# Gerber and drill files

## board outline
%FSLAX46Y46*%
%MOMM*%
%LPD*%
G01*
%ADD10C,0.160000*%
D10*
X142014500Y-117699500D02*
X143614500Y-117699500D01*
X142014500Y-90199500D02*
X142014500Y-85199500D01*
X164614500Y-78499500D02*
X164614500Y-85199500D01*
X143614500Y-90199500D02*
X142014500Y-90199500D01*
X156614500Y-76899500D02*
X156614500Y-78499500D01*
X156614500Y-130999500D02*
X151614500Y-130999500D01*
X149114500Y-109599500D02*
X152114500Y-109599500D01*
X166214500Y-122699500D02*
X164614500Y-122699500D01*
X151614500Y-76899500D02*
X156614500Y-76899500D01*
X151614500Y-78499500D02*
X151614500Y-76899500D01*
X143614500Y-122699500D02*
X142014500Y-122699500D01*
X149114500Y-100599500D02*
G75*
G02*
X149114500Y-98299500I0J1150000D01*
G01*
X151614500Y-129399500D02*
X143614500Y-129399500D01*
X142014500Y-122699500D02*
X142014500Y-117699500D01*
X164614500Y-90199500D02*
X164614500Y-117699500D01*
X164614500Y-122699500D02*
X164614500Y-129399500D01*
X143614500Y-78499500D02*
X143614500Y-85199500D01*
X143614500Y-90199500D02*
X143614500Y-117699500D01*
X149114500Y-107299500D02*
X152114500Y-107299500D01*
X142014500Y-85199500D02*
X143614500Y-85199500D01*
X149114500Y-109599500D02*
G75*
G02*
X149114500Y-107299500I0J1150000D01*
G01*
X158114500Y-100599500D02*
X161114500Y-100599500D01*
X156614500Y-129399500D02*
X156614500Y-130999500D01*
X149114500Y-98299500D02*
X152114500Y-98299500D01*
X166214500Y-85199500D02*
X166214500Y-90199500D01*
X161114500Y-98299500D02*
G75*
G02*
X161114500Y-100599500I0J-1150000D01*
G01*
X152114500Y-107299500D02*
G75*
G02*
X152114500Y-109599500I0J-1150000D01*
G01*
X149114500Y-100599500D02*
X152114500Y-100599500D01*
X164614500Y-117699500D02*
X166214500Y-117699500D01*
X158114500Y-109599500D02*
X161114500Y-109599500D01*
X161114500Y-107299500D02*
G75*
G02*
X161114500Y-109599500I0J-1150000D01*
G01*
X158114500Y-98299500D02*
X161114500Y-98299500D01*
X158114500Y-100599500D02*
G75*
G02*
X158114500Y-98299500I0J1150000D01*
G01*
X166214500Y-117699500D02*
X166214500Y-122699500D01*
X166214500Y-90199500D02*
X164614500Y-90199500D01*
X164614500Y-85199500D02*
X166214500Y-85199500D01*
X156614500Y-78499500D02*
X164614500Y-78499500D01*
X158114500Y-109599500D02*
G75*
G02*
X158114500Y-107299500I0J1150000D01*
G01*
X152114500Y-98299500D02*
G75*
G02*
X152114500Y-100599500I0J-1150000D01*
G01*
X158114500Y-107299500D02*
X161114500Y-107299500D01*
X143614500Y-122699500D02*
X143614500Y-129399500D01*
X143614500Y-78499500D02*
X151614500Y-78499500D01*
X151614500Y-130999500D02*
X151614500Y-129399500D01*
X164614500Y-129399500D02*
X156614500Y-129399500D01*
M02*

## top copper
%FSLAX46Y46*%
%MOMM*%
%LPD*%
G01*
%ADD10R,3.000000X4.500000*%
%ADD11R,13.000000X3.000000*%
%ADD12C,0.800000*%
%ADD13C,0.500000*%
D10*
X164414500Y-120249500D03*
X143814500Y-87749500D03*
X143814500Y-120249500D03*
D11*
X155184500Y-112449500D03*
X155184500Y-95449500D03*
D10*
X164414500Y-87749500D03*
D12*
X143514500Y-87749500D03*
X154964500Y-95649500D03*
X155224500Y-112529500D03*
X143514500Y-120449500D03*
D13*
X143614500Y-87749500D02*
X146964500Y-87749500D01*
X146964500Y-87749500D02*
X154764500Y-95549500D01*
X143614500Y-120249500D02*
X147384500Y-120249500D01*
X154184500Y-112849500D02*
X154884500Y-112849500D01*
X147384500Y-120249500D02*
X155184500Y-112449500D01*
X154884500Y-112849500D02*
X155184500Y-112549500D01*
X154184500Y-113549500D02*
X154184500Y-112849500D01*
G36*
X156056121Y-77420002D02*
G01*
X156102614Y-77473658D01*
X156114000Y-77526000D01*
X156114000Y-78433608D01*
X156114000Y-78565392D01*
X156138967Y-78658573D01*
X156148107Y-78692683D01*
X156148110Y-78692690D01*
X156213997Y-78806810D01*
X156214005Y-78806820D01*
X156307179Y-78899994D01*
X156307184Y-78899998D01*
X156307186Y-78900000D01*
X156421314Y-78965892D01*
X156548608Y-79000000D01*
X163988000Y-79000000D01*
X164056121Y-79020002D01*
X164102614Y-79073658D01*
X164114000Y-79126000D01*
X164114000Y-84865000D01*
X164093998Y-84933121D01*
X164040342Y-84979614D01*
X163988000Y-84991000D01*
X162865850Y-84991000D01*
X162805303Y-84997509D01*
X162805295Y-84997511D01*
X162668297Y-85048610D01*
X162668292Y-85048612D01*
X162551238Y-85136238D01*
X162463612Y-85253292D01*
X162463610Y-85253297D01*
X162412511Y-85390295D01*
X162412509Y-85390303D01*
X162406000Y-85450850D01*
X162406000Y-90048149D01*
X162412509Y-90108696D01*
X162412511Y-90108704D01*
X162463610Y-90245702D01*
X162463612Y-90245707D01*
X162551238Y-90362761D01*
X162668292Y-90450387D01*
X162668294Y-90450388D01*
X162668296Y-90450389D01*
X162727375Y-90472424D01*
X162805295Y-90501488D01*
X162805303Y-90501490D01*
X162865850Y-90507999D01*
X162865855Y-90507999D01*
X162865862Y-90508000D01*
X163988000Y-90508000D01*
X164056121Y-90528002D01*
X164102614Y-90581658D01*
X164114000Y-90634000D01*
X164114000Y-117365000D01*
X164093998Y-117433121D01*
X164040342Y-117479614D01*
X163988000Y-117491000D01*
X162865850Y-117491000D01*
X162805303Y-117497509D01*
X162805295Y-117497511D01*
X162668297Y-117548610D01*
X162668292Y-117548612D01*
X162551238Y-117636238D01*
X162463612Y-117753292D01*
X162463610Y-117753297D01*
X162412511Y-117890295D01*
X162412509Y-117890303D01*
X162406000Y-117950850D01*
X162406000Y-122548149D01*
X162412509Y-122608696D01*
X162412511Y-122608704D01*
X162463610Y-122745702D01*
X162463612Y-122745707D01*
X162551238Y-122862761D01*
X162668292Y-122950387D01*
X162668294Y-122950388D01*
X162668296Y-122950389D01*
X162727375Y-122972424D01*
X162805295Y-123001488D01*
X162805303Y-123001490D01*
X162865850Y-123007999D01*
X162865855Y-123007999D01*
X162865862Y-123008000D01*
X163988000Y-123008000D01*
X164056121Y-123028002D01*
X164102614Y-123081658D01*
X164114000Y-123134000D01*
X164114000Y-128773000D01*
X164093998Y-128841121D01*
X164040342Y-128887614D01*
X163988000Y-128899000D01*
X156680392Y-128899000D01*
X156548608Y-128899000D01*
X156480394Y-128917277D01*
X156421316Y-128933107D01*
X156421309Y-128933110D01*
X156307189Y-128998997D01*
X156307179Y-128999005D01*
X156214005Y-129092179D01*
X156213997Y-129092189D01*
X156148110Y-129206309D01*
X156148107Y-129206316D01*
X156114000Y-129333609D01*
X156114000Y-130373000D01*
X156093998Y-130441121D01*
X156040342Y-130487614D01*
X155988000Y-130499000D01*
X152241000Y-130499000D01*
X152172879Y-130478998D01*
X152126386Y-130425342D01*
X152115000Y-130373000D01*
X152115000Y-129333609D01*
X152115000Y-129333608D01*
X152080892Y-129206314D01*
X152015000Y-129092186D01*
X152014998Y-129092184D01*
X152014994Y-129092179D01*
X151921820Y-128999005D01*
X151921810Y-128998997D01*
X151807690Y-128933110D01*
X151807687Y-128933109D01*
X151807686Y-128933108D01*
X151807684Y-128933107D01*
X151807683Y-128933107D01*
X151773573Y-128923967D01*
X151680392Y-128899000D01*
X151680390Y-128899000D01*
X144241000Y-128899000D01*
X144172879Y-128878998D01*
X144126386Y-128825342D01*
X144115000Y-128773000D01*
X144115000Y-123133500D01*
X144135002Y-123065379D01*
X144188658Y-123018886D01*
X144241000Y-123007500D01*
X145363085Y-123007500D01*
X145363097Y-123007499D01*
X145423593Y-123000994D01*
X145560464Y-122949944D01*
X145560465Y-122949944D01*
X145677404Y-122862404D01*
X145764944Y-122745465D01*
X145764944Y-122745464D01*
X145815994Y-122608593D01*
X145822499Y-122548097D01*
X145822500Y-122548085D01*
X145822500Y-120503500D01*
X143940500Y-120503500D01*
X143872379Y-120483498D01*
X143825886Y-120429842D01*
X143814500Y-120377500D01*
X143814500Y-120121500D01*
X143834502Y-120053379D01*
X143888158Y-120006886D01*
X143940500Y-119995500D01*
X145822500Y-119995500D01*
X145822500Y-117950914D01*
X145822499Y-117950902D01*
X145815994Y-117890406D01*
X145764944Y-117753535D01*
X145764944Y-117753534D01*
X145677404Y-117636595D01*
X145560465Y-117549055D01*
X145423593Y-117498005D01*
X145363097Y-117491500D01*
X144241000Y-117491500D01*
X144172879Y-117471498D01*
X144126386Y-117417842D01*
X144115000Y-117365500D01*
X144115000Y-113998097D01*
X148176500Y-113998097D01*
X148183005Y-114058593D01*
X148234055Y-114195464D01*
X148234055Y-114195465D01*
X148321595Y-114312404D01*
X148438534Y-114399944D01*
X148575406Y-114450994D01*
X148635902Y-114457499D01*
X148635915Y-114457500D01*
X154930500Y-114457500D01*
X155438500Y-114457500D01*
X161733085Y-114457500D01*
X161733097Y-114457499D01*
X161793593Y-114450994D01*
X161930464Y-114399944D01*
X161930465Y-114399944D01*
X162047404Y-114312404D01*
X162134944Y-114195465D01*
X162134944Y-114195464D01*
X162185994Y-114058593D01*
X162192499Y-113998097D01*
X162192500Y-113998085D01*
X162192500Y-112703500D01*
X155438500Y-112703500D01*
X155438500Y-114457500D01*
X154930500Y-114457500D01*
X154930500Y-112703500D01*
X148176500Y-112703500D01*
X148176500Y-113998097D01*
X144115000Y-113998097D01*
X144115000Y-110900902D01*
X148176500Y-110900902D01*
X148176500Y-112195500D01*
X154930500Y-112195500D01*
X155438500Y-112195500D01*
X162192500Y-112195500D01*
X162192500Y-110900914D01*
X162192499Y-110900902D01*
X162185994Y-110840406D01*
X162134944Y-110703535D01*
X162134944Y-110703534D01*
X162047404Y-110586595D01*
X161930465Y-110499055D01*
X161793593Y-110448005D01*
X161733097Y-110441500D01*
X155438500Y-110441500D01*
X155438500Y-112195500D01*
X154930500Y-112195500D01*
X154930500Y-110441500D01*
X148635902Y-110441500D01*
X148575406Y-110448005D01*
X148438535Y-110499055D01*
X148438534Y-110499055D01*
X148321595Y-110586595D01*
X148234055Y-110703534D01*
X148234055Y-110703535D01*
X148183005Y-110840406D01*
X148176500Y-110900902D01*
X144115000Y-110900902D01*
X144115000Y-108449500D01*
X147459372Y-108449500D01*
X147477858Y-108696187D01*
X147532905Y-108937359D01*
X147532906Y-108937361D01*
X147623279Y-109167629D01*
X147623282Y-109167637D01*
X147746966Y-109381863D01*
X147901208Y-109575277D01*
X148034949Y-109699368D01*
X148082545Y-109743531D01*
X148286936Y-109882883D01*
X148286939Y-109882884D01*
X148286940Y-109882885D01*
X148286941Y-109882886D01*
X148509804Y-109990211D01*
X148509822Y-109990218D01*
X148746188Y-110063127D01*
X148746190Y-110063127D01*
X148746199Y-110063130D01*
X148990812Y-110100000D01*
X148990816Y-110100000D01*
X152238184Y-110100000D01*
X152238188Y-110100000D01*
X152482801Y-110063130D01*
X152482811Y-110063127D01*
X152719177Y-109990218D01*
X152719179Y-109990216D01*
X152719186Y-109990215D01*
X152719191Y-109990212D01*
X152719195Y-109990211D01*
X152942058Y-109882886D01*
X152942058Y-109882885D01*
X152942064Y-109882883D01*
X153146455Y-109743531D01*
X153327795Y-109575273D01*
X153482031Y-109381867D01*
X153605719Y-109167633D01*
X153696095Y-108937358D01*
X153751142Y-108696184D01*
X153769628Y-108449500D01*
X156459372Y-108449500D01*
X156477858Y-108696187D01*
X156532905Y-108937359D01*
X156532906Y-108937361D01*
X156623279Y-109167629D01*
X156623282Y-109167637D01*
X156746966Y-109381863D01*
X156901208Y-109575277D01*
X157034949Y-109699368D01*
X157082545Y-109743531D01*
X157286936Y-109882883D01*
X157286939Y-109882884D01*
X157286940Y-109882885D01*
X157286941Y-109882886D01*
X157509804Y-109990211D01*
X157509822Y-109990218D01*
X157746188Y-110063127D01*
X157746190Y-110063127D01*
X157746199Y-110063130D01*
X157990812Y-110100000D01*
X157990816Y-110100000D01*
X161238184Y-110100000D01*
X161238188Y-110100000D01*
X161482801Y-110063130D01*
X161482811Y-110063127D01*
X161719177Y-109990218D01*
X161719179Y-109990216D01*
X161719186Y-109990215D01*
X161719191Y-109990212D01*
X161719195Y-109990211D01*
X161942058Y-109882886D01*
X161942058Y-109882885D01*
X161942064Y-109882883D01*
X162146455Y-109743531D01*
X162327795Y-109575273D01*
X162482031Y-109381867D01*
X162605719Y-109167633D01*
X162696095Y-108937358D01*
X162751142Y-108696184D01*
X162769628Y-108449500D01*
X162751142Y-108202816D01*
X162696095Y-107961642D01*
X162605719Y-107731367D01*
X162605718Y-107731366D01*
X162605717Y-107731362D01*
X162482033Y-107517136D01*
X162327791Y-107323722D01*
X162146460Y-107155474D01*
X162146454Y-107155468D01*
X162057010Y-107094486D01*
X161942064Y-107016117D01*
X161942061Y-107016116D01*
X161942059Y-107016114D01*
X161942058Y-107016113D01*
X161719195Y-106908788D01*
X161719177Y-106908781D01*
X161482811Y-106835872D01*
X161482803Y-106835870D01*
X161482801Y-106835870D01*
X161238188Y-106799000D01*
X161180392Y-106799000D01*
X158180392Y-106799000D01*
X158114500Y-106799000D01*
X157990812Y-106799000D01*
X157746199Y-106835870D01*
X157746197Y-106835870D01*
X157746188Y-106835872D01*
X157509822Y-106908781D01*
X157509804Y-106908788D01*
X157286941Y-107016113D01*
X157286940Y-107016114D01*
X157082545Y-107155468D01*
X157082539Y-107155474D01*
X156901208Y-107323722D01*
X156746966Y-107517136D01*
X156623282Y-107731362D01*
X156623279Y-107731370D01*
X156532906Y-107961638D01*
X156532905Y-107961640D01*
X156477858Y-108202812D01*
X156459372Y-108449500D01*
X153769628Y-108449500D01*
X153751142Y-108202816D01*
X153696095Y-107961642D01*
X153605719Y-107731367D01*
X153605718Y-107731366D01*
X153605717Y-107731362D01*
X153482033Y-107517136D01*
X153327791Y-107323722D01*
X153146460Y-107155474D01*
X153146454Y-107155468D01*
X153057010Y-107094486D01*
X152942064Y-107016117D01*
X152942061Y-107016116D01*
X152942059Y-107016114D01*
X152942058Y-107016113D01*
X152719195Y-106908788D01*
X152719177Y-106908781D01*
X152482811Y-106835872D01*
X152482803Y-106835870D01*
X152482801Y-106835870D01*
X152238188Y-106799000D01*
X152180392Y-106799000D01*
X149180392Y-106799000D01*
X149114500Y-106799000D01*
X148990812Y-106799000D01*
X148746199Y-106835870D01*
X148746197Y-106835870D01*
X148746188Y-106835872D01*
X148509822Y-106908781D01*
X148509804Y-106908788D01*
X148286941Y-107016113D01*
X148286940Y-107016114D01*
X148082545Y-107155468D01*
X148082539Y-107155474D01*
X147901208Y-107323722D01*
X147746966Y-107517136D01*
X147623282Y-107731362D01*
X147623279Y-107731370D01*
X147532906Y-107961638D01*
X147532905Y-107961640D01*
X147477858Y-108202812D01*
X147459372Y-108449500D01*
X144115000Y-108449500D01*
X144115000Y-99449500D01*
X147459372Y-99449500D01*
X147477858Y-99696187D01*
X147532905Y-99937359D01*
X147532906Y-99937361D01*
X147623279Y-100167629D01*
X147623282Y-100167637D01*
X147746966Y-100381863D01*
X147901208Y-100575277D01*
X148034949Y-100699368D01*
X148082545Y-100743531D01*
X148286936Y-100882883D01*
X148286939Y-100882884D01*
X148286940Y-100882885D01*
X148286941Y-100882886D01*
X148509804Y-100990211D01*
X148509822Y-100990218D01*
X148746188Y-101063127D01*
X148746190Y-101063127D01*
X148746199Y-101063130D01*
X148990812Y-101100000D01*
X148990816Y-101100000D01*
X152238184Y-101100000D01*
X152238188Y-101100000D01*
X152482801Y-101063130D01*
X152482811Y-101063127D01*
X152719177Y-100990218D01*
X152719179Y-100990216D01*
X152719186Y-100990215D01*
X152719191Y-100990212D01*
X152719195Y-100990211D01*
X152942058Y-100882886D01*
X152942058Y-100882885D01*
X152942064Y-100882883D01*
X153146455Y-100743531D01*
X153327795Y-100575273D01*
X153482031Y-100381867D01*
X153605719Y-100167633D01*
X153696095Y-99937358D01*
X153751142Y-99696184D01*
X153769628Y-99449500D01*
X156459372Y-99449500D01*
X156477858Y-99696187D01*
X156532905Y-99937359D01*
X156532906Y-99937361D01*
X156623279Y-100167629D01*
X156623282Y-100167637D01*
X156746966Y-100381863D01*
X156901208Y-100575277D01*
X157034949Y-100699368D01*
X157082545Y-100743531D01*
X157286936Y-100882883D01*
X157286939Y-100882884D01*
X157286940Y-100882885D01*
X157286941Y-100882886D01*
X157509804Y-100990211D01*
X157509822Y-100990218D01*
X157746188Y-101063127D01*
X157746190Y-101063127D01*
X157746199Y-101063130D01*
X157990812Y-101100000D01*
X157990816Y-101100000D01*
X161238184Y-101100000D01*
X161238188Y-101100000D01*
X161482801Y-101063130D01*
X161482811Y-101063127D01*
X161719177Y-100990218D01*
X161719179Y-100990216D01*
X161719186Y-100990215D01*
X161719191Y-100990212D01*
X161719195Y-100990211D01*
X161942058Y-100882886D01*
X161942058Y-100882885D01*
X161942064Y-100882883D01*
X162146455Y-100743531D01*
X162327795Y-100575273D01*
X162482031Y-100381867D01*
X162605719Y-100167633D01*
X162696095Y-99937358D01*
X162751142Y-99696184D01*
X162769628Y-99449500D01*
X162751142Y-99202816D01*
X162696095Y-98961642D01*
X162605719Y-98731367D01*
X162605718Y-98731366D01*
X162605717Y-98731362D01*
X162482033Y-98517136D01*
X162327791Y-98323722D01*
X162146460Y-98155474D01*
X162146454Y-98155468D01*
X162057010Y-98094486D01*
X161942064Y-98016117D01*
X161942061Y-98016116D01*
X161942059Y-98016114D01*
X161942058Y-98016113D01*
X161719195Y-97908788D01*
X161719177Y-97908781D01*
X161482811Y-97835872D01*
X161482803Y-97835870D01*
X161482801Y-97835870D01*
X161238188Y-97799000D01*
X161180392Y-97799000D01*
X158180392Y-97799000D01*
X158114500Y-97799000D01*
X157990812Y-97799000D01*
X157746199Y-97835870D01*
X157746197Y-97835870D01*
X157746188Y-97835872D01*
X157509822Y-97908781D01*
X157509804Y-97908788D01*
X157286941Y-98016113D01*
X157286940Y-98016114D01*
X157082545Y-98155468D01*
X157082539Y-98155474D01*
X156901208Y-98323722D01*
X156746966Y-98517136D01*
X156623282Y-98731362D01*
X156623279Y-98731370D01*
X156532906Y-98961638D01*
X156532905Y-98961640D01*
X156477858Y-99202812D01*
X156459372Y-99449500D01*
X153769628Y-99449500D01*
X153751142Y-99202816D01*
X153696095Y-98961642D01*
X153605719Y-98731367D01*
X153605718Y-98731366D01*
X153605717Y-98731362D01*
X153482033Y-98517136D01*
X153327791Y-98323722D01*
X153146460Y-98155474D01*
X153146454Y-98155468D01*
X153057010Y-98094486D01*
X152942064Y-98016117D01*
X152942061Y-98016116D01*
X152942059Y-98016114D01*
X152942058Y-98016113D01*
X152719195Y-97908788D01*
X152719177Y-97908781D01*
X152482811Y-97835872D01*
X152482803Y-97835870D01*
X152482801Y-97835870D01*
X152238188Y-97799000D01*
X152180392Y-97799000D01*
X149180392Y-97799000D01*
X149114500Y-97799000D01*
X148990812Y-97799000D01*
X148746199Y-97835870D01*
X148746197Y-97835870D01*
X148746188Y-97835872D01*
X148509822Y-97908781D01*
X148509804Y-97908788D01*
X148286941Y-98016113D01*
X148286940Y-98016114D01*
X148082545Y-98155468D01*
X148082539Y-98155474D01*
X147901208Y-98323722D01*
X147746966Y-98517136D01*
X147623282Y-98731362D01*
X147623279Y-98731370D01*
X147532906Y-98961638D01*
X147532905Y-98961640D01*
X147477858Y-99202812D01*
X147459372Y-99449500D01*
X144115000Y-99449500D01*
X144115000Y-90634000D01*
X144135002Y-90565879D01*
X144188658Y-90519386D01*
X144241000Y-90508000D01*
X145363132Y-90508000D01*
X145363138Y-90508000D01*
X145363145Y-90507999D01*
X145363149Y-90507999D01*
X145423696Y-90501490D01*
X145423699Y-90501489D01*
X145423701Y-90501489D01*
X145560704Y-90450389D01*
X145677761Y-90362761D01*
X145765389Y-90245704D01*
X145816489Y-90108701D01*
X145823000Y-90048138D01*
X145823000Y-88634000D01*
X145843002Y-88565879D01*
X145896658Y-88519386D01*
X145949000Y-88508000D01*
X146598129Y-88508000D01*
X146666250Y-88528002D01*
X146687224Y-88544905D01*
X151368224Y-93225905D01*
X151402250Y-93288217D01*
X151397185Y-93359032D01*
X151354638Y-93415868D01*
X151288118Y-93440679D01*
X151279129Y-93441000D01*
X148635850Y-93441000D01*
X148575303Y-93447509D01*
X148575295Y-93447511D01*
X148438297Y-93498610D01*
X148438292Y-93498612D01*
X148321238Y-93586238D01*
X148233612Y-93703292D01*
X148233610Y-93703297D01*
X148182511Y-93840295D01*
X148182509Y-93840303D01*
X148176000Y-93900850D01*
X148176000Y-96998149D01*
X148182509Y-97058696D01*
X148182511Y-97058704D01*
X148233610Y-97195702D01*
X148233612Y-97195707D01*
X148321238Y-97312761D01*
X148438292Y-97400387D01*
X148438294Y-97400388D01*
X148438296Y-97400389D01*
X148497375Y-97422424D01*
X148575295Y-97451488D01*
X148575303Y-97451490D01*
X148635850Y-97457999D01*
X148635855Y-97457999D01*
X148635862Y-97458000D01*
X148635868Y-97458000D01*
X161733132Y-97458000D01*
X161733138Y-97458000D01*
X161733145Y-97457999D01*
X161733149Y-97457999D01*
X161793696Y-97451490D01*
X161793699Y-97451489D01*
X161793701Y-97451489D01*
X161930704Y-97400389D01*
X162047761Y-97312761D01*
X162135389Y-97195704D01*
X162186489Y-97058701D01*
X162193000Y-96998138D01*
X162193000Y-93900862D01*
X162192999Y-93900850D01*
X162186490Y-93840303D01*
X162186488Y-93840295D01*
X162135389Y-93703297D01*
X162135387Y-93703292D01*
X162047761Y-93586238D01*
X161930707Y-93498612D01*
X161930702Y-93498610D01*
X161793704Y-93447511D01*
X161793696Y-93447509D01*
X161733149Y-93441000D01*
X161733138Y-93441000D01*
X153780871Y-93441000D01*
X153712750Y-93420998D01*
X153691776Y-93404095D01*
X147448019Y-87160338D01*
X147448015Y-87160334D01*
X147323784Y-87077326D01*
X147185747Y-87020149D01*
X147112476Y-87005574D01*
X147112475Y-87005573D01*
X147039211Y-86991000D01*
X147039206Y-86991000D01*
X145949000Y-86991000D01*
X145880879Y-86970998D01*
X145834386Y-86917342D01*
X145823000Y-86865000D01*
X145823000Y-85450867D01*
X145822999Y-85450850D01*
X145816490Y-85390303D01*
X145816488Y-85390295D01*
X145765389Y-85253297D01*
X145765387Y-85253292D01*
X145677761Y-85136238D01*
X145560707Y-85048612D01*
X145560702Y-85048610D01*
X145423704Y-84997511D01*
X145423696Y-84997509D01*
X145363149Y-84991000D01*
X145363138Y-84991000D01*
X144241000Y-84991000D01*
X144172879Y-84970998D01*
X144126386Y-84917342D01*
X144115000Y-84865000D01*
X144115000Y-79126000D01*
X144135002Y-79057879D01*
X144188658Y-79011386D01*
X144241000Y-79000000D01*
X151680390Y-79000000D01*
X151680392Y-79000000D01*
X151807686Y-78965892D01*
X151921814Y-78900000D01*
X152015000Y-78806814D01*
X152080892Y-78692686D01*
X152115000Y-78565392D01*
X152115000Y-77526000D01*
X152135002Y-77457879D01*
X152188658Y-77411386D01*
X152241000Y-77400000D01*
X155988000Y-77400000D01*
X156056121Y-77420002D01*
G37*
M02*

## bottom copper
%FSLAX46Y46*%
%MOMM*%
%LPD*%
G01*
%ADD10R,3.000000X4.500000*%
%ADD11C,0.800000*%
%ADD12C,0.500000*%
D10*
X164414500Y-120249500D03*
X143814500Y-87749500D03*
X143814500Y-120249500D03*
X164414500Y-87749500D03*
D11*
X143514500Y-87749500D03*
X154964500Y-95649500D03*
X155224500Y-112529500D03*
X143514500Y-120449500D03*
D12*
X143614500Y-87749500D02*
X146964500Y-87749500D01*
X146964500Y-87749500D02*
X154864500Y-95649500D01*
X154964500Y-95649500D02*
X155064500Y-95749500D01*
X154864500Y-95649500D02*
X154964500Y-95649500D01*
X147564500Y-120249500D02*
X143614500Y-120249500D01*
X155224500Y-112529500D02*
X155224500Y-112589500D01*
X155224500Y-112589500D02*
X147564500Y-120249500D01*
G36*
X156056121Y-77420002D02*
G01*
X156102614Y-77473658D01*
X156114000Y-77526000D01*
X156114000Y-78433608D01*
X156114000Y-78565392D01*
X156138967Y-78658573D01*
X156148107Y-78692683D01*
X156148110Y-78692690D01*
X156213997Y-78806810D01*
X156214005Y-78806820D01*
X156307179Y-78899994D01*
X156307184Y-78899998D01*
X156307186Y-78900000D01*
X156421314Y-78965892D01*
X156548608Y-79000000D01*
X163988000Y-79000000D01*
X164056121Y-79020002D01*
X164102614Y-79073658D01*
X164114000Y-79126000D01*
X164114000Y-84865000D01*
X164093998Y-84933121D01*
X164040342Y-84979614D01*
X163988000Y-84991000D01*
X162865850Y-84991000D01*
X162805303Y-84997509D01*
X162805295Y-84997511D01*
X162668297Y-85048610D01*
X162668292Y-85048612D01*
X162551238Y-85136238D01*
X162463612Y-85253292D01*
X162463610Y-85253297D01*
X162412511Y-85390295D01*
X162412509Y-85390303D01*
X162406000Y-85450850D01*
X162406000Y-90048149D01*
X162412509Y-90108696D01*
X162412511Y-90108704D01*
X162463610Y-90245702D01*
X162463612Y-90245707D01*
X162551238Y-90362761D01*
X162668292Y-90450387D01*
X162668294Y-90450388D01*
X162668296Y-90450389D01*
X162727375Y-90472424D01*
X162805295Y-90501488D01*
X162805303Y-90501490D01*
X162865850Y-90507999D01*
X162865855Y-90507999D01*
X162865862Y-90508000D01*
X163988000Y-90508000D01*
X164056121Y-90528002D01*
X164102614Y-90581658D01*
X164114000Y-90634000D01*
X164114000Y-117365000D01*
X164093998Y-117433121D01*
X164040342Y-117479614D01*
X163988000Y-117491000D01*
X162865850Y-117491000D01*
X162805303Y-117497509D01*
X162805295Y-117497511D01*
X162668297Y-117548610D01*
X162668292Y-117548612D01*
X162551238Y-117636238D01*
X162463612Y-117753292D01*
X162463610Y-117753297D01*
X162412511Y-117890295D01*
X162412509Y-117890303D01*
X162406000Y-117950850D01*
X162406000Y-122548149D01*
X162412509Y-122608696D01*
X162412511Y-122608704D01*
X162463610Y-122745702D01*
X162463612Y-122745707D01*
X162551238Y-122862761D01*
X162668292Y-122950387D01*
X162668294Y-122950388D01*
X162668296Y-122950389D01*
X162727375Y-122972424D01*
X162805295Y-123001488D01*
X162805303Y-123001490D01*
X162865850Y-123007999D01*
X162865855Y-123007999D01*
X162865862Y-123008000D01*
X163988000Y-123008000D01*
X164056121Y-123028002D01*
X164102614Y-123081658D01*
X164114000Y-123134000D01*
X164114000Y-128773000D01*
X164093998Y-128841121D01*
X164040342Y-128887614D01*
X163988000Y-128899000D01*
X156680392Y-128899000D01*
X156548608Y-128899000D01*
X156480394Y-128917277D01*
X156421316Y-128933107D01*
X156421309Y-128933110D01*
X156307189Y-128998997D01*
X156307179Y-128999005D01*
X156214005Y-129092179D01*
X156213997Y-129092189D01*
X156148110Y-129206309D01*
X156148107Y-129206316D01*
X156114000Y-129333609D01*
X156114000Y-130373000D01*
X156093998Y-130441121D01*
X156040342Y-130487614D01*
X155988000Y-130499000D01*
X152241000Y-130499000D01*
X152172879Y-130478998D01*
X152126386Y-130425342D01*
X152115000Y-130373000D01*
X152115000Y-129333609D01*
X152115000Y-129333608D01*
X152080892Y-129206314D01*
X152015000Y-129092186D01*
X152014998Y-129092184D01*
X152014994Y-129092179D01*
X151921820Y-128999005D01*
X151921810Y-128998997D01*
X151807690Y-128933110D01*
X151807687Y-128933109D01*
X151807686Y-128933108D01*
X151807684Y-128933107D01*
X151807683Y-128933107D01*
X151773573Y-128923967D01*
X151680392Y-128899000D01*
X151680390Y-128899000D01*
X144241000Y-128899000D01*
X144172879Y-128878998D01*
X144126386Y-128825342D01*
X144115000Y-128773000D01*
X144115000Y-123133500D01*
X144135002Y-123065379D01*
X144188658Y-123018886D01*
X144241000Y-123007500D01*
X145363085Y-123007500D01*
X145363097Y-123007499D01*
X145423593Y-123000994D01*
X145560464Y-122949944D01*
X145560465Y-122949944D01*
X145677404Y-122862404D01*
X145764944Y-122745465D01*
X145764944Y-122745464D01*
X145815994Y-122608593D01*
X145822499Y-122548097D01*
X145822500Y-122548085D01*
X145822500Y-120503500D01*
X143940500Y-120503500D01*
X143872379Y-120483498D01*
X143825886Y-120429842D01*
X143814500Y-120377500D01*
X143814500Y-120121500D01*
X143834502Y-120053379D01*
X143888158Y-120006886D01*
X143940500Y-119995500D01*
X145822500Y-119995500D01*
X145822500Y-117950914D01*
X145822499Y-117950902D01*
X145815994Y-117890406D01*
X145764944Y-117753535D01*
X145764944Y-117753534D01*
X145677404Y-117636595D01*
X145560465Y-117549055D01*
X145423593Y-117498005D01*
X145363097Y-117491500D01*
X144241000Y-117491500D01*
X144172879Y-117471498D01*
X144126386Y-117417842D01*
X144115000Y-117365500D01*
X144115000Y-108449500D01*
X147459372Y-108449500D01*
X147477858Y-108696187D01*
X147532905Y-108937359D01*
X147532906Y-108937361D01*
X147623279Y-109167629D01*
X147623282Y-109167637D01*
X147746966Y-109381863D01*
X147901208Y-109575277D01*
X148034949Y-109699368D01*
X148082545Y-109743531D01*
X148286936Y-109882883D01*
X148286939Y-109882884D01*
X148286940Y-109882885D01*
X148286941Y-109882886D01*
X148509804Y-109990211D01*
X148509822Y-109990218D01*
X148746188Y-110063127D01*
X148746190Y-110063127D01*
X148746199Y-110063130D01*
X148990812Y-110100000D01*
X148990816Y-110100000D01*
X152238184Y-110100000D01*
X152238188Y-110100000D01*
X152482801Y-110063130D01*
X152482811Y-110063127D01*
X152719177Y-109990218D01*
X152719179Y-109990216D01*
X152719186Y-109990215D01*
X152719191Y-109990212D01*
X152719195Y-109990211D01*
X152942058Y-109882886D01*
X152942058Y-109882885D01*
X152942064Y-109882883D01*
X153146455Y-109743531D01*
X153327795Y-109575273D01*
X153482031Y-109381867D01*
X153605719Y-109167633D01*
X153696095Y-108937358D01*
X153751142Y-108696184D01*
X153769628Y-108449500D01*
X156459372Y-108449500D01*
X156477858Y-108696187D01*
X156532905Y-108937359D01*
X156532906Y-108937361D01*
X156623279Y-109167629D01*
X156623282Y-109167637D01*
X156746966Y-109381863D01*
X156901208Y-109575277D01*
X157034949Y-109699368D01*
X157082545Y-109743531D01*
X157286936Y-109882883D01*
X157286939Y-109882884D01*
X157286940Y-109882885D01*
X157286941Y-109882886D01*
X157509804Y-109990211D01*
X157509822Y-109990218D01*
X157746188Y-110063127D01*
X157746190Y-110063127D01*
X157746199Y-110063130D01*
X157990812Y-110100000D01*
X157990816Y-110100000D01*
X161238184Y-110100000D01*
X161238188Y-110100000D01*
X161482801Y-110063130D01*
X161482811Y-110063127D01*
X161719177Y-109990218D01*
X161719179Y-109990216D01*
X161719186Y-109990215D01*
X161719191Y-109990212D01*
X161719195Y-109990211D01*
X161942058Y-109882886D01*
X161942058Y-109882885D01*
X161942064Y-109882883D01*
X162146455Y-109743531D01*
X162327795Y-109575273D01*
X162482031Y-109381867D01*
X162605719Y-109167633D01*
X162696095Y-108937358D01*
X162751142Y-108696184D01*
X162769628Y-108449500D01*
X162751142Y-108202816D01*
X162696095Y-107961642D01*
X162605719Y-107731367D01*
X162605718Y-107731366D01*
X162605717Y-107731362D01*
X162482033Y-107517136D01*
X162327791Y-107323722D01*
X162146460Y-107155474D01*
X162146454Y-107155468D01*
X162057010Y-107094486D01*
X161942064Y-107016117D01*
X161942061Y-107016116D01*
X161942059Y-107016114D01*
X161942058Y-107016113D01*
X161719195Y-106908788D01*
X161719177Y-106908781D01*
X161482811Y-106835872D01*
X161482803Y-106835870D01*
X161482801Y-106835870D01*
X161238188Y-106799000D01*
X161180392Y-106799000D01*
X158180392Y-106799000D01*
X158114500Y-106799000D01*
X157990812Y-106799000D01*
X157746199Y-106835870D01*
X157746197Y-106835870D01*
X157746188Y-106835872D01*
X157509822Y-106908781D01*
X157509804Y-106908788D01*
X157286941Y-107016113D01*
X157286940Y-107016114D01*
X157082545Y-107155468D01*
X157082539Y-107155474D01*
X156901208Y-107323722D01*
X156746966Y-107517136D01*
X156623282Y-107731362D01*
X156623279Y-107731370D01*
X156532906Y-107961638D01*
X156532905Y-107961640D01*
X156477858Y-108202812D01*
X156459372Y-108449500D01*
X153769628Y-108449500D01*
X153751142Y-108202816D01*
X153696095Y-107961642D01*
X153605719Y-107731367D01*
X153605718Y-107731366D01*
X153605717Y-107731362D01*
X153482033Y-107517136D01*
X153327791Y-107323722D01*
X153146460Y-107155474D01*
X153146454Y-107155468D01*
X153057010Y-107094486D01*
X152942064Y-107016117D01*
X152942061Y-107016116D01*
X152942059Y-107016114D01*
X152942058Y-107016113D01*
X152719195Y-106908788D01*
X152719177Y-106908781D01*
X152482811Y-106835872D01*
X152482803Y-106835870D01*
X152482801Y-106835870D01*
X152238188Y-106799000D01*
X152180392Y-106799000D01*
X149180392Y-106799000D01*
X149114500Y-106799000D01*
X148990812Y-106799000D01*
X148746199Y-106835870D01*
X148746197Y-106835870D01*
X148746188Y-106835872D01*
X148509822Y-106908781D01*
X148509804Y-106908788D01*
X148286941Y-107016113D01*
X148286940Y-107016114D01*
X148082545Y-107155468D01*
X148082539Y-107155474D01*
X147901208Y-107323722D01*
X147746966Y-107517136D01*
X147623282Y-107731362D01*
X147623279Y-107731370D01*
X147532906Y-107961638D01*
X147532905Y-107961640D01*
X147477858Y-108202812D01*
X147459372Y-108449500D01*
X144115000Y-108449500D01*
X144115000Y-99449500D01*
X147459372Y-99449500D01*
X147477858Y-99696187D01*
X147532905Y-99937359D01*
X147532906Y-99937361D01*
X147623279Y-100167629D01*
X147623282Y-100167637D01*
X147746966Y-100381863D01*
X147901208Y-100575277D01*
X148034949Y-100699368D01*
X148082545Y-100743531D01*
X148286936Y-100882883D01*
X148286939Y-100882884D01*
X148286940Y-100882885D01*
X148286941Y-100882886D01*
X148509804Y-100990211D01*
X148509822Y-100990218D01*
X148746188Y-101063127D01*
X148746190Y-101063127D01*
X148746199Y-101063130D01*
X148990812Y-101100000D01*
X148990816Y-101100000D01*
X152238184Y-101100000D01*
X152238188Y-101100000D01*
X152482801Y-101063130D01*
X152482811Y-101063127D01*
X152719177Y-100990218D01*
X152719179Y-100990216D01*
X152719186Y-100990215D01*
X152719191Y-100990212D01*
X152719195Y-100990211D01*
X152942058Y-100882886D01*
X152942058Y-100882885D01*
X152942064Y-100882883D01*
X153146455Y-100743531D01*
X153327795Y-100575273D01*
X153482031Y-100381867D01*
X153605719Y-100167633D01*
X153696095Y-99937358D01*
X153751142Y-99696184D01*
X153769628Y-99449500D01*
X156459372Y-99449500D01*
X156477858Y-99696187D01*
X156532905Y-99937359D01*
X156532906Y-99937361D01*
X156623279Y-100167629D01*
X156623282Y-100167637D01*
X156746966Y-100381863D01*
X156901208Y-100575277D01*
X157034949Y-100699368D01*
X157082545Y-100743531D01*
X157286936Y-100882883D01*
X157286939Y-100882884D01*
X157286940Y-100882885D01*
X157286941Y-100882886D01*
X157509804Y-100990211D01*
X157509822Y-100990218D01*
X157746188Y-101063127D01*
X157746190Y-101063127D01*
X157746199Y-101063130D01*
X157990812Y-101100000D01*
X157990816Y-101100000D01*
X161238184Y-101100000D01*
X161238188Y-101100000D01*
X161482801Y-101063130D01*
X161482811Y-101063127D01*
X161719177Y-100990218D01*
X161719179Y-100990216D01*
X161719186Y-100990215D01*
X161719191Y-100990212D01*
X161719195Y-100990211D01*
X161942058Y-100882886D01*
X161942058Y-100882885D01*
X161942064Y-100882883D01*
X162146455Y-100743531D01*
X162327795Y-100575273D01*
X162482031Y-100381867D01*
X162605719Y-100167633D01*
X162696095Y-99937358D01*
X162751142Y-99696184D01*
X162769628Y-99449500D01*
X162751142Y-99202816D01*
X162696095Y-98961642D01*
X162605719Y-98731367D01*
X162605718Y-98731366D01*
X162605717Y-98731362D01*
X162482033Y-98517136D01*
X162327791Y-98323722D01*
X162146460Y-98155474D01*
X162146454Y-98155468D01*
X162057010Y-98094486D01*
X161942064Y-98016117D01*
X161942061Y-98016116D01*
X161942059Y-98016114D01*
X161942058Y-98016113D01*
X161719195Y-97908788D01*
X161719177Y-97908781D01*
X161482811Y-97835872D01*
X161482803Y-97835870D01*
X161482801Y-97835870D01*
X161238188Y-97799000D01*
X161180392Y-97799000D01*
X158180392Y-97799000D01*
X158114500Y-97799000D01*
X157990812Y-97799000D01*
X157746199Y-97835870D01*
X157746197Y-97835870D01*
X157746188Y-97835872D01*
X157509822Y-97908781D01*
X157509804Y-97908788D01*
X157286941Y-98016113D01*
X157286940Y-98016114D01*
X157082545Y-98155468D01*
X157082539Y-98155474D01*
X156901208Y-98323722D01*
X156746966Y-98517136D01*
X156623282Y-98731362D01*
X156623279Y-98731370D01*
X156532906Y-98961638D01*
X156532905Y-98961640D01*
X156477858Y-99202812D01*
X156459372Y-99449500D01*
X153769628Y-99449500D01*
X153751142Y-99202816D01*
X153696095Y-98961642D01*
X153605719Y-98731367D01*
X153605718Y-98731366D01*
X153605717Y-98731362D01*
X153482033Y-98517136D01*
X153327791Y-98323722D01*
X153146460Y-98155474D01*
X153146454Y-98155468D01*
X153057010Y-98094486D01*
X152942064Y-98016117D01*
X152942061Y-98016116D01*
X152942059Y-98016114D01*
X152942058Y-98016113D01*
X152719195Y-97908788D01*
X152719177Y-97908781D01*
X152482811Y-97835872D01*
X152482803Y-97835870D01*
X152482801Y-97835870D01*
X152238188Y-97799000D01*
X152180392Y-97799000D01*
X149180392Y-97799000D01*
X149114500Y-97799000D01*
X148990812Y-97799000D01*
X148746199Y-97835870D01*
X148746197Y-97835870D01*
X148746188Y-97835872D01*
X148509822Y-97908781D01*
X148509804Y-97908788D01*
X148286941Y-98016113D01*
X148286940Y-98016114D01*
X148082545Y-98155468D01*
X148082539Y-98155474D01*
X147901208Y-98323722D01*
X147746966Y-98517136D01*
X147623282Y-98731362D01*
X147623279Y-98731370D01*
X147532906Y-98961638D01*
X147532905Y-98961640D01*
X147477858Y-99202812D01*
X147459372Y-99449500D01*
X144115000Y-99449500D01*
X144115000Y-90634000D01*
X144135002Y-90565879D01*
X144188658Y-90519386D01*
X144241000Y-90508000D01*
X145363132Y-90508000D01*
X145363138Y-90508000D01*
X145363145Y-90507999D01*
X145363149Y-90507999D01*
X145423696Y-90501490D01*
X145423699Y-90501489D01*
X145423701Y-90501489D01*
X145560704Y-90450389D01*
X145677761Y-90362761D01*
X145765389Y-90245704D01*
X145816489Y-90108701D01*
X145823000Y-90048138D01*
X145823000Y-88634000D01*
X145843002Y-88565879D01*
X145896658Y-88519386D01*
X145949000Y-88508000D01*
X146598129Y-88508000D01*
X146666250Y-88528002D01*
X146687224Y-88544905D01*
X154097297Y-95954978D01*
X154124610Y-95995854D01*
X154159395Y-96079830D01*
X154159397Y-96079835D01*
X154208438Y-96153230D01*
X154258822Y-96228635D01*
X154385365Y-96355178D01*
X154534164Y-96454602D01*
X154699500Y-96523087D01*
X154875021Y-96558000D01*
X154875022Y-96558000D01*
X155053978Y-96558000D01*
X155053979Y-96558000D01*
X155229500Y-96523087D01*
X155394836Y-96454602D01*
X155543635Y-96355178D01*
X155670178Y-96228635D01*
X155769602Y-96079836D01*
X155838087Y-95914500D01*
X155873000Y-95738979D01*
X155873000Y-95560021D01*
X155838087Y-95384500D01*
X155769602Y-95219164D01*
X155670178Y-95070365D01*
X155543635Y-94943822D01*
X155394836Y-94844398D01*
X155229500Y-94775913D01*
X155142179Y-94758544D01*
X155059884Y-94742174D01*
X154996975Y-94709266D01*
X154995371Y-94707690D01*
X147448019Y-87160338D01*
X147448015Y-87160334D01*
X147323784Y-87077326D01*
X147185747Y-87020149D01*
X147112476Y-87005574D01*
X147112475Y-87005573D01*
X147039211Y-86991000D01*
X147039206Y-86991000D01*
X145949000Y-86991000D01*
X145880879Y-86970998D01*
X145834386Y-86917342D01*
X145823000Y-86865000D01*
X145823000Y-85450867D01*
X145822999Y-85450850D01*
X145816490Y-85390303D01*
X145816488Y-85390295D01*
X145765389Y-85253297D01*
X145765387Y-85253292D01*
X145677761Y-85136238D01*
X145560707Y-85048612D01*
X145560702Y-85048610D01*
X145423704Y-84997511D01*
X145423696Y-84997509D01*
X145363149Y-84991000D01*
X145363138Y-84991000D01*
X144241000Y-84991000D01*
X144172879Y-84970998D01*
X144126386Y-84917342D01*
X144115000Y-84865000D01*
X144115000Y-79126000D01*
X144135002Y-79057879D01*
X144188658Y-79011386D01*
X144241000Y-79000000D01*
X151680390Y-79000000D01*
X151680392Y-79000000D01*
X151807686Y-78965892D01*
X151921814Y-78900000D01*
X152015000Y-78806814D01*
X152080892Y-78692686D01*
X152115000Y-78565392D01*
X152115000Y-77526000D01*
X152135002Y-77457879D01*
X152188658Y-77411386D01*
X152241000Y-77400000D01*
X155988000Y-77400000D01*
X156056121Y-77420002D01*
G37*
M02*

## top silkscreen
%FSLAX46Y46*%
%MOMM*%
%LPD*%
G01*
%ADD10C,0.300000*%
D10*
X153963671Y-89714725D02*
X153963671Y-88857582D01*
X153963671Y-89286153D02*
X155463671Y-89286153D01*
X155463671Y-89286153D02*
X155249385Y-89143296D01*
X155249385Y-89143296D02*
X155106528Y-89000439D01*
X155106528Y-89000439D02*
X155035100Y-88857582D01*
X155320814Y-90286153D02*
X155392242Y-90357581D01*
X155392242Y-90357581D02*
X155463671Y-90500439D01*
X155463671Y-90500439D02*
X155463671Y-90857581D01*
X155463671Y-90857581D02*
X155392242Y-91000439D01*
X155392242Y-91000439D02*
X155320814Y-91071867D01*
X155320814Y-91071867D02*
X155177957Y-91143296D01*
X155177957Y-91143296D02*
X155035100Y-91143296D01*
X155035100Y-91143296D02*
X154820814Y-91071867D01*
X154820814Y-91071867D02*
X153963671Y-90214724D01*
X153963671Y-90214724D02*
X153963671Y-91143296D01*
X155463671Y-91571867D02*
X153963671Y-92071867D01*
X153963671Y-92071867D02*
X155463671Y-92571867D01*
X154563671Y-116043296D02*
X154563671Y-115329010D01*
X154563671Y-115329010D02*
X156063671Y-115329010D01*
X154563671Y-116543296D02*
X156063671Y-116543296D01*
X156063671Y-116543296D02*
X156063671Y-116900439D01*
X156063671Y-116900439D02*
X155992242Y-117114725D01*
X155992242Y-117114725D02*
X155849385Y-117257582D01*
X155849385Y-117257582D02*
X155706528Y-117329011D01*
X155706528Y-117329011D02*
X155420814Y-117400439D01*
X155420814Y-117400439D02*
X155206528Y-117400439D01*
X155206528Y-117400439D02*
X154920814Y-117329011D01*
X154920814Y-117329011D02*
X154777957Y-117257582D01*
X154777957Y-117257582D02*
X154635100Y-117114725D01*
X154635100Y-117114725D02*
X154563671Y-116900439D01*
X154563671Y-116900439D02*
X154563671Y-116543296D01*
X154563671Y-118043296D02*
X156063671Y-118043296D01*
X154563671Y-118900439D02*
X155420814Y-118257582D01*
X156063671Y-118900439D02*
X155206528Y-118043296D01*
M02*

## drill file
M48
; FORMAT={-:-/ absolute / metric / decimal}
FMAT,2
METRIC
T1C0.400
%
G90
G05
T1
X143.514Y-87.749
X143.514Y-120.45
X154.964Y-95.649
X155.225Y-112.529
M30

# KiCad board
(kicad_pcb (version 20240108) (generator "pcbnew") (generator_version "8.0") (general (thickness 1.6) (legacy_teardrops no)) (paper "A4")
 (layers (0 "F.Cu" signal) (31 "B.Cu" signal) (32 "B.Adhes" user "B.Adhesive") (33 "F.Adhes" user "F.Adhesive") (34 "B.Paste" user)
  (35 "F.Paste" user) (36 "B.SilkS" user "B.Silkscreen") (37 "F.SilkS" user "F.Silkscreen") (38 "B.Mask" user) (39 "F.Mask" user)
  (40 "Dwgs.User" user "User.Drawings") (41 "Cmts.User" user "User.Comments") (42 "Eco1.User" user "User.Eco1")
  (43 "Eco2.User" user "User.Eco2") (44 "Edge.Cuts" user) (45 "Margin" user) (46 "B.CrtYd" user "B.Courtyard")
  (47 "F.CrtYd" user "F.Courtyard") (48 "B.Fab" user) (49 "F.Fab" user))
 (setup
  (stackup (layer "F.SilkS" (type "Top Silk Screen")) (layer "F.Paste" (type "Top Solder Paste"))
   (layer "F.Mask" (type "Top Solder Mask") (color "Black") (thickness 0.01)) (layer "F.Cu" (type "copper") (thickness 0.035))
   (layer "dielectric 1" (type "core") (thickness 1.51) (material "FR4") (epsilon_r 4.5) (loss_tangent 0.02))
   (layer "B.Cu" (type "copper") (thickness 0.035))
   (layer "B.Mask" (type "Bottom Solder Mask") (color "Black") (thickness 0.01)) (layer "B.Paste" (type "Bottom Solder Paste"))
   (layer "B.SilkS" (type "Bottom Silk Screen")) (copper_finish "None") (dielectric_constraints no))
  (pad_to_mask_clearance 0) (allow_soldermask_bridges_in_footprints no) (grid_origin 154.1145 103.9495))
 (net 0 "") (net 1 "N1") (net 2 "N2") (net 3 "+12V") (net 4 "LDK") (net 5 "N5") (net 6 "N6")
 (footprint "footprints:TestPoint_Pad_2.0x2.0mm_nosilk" (layer "F.Cu") (at 164.4145 120.2495 90)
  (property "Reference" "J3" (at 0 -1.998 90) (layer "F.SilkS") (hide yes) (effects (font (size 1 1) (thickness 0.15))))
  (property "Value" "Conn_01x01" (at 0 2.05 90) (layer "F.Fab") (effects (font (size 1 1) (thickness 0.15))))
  (pad "1" smd rect (at 0 0 90) (size 4.5 3) (layers "F.Cu" "F.Mask") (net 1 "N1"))
  (pad "1" smd rect (at 0 0 90) (size 4.5 3) (layers "B.Cu" "B.Mask") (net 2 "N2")))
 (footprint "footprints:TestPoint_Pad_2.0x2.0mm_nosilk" (layer "F.Cu") (at 143.8145 87.7495 90)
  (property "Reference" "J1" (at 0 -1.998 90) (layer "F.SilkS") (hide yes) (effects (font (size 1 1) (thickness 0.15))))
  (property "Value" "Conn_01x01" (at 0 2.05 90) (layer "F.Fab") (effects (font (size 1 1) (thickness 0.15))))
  (pad "1" smd rect (at 0 0 90) (size 4.5 3) (layers "F.Cu" "F.Mask") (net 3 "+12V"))
  (pad "1" smd rect (at 0 0 90) (size 4.5 3) (layers "B.Cu" "B.Mask") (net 3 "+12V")))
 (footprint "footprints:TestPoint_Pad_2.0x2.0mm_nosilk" (layer "F.Cu") (at 143.8145 120.2495 -90)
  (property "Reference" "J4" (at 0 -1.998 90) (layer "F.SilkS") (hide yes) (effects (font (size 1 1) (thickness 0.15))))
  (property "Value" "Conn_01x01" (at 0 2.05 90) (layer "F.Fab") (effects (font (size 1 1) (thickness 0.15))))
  (pad "1" smd rect (at 0 0 270) (size 4.5 3) (layers "F.Cu" "F.Mask") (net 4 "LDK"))
  (pad "1" smd rect (at 0 0 270) (size 4.5 3) (layers "B.Cu" "B.Mask") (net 4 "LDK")))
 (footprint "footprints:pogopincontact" (layer "F.Cu") (at 155.1845 103.9495 90)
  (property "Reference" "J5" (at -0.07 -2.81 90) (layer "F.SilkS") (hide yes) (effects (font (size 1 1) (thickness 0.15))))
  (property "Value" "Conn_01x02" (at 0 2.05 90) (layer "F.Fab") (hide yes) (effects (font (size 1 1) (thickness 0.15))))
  (pad "1" smd rect (at -8.5 0 90) (size 3 13) (layers "F.Cu" "F.Mask") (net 4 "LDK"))
  (pad "2" smd rect (at 8.5 0 90) (size 3 13) (layers "F.Cu" "F.Mask") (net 3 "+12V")))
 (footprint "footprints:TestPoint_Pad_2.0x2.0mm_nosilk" (layer "F.Cu") (at 164.4145 87.7495 90)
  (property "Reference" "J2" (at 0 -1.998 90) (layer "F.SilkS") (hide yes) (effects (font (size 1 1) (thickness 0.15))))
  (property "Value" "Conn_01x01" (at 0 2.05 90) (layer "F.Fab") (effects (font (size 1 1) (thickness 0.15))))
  (pad "1" smd rect (at 0 0 90) (size 4.5 3) (layers "F.Cu" "F.Mask") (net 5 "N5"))
  (pad "1" smd rect (at 0 0 90) (size 4.5 3) (layers "B.Cu" "B.Mask") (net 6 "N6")))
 (gr_line (start 142.0145 117.6995) (end 143.6145 117.6995) (stroke (width 0.16) (type solid)) (layer "Edge.Cuts"))
 (gr_line (start 142.0145 90.1995) (end 142.0145 85.1995) (stroke (width 0.16) (type solid)) (layer "Edge.Cuts"))
 (gr_line (start 164.6145 78.4995) (end 164.6145 85.1995) (stroke (width 0.16) (type solid)) (layer "Edge.Cuts"))
 (gr_line (start 143.6145 90.1995) (end 142.0145 90.1995) (stroke (width 0.16) (type solid)) (layer "Edge.Cuts"))
 (gr_line (start 156.6145 76.8995) (end 156.6145 78.4995) (stroke (width 0.16) (type solid)) (layer "Edge.Cuts"))
 (gr_line (start 156.6145 130.9995) (end 151.6145 130.9995) (stroke (width 0.16) (type solid)) (layer "Edge.Cuts"))
 (gr_line (start 149.1145 109.5995) (end 152.1145 109.5995) (stroke (width 0.16) (type solid)) (layer "Edge.Cuts"))
 (gr_line (start 166.2145 122.6995) (end 164.6145 122.6995) (stroke (width 0.16) (type solid)) (layer "Edge.Cuts"))
 (gr_line (start 151.6145 76.8995) (end 156.6145 76.8995) (stroke (width 0.16) (type solid)) (layer "Edge.Cuts"))
 (gr_line (start 151.6145 78.4995) (end 151.6145 76.8995) (stroke (width 0.16) (type solid)) (layer "Edge.Cuts"))
 (gr_line (start 143.6145 122.6995) (end 142.0145 122.6995) (stroke (width 0.16) (type solid)) (layer "Edge.Cuts"))
 (gr_arc (start 149.1145 100.5995) (mid 147.9645 99.4495) (end 149.1145 98.2995) (stroke (width 0.16) (type solid)) (layer "Edge.Cuts"))
 (gr_line (start 151.6145 129.3995) (end 143.6145 129.3995) (stroke (width 0.16) (type solid)) (layer "Edge.Cuts"))
 (gr_line (start 142.0145 122.6995) (end 142.0145 117.6995) (stroke (width 0.16) (type solid)) (layer "Edge.Cuts"))
 (gr_line (start 164.6145 90.1995) (end 164.6145 117.6995) (stroke (width 0.16) (type solid)) (layer "Edge.Cuts"))
 (gr_line (start 164.6145 122.6995) (end 164.6145 129.3995) (stroke (width 0.16) (type solid)) (layer "Edge.Cuts"))
 (gr_line (start 143.6145 78.4995) (end 143.6145 85.1995) (stroke (width 0.16) (type solid)) (layer "Edge.Cuts"))
 (gr_line (start 143.6145 90.1995) (end 143.6145 117.6995) (stroke (width 0.16) (type solid)) (layer "Edge.Cuts"))
 (gr_line (start 149.1145 107.2995) (end 152.1145 107.2995) (stroke (width 0.16) (type solid)) (layer "Edge.Cuts"))
 (gr_line (start 142.0145 85.1995) (end 143.6145 85.1995) (stroke (width 0.16) (type solid)) (layer "Edge.Cuts"))
 (gr_arc (start 149.1145 109.5995) (mid 147.9645 108.4495) (end 149.1145 107.2995) (stroke (width 0.16) (type solid)) (layer "Edge.Cuts"))
 (gr_line (start 158.1145 100.5995) (end 161.1145 100.5995) (stroke (width 0.16) (type solid)) (layer "Edge.Cuts"))
 (gr_line (start 156.6145 129.3995) (end 156.6145 130.9995) (stroke (width 0.16) (type solid)) (layer "Edge.Cuts"))
 (gr_line (start 149.1145 98.2995) (end 152.1145 98.2995) (stroke (width 0.16) (type solid)) (layer "Edge.Cuts"))
 (gr_line (start 166.2145 85.1995) (end 166.2145 90.1995) (stroke (width 0.16) (type solid)) (layer "Edge.Cuts"))
 (gr_arc (start 161.1145 98.2995) (mid 162.2645 99.4495) (end 161.1145 100.5995) (stroke (width 0.16) (type solid)) (layer "Edge.Cuts"))
 (gr_arc (start 152.1145 107.2995) (mid 153.2645 108.4495) (end 152.1145 109.5995) (stroke (width 0.16) (type solid)) (layer "Edge.Cuts"))
 (gr_line (start 149.1145 100.5995) (end 152.1145 100.5995) (stroke (width 0.16) (type solid)) (layer "Edge.Cuts"))
 (gr_line (start 164.6145 117.6995) (end 166.2145 117.6995) (stroke (width 0.16) (type solid)) (layer "Edge.Cuts"))
 (gr_line (start 158.1145 109.5995) (end 161.1145 109.5995) (stroke (width 0.16) (type solid)) (layer "Edge.Cuts"))
 (gr_arc (start 161.1145 107.2995) (mid 162.2645 108.4495) (end 161.1145 109.5995) (stroke (width 0.16) (type solid)) (layer "Edge.Cuts"))
 (gr_line (start 158.1145 98.2995) (end 161.1145 98.2995) (stroke (width 0.16) (type solid)) (layer "Edge.Cuts"))
 (gr_arc (start 158.1145 100.5995) (mid 156.9645 99.4495) (end 158.1145 98.2995) (stroke (width 0.16) (type solid)) (layer "Edge.Cuts"))
 (gr_line (start 166.2145 117.6995) (end 166.2145 122.6995) (stroke (width 0.16) (type solid)) (layer "Edge.Cuts"))
 (gr_line (start 166.2145 90.1995) (end 164.6145 90.1995) (stroke (width 0.16) (type solid)) (layer "Edge.Cuts"))
 (gr_line (start 164.6145 85.1995) (end 166.2145 85.1995) (stroke (width 0.16) (type solid)) (layer "Edge.Cuts"))
 (gr_line (start 156.6145 78.4995) (end 164.6145 78.4995) (stroke (width 0.16) (type solid)) (layer "Edge.Cuts"))
 (gr_arc (start 158.1145 109.5995) (mid 156.9645 108.4495) (end 158.1145 107.2995) (stroke (width 0.16) (type solid)) (layer "Edge.Cuts"))
 (gr_arc (start 152.1145 98.2995) (mid 153.2645 99.4495) (end 152.1145 100.5995) (stroke (width 0.16) (type solid)) (layer "Edge.Cuts"))
 (gr_line (start 158.1145 107.2995) (end 161.1145 107.2995) (stroke (width 0.16) (type solid)) (layer "Edge.Cuts"))
 (gr_line (start 143.6145 122.6995) (end 143.6145 129.3995) (stroke (width 0.16) (type solid)) (layer "Edge.Cuts"))
 (gr_line (start 143.6145 78.4995) (end 151.6145 78.4995) (stroke (width 0.16) (type solid)) (layer "Edge.Cuts"))
 (gr_line (start 151.6145 130.9995) (end 151.6145 129.3995) (stroke (width 0.16) (type solid)) (layer "Edge.Cuts"))
 (gr_line (start 164.6145 129.3995) (end 156.6145 129.3995) (stroke (width 0.16) (type solid)) (layer "Edge.Cuts"))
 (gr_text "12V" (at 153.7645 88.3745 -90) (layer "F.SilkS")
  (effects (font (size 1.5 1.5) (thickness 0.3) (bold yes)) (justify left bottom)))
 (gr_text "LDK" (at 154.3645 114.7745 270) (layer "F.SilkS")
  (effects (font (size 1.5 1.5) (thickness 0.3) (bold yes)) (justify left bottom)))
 (segment (start 143.6145 87.7495) (end 146.9645 87.7495) (width 0.5) (layer "F.Cu") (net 3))
 (segment (start 146.9645 87.7495) (end 154.7645 95.5495) (width 0.5) (layer "F.Cu") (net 3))
 (via (at 143.5145 87.7495) (size 0.8) (drill 0.4) (layers "F.Cu" "B.Cu") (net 3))
 (via (at 154.9645 95.6495) (size 0.8) (drill 0.4) (layers "F.Cu" "B.Cu") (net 3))
 (segment (start 143.6145 87.7495) (end 146.9645 87.7495) (width 0.5) (layer "B.Cu") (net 3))
 (segment (start 146.9645 87.7495) (end 154.8645 95.6495) (width 0.5) (layer "B.Cu") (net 3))
 (segment (start 154.9645 95.6495) (end 155.0645 95.7495) (width 0.5) (layer "B.Cu") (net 3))
 (segment (start 154.8645 95.6495) (end 154.9645 95.6495) (width 0.5) (layer "B.Cu") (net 3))
 (segment (start 143.6145 120.2495) (end 147.3845 120.2495) (width 0.5) (layer "F.Cu") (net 4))
 (segment (start 154.1845 112.8495) (end 154.8845 112.8495) (width 0.5) (layer "F.Cu") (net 4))
 (segment (start 147.3845 120.2495) (end 155.1845 112.4495) (width 0.5) (layer "F.Cu") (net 4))
 (segment (start 154.8845 112.8495) (end 155.1845 112.5495) (width 0.5) (layer "F.Cu") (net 4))
 (segment (start 154.1845 113.5495) (end 154.1845 112.8495) (width 0.5) (layer "F.Cu") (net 4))
 (via (at 155.2245 112.5295) (size 0.8) (drill 0.4) (layers "F.Cu" "B.Cu") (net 4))
 (via (at 143.5145 120.4495) (size 0.8) (drill 0.4) (layers "F.Cu" "B.Cu") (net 4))
 (segment (start 147.5645 120.2495) (end 143.6145 120.2495) (width 0.5) (layer "B.Cu") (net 4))
 (segment (start 155.2245 112.5295) (end 155.2245 112.5895) (width 0.5) (layer "B.Cu") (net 4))
 (segment (start 155.2245 112.5895) (end 147.5645 120.2495) (width 0.5) (layer "B.Cu") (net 4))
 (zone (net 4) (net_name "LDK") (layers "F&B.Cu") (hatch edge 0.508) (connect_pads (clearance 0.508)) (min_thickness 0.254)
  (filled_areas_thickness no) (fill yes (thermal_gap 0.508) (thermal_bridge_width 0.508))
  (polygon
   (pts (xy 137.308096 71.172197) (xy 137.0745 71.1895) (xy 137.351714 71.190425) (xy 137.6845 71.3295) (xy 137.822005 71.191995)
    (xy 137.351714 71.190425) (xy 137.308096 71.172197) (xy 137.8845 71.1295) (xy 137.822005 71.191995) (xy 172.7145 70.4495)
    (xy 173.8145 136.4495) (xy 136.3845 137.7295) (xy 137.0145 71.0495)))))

